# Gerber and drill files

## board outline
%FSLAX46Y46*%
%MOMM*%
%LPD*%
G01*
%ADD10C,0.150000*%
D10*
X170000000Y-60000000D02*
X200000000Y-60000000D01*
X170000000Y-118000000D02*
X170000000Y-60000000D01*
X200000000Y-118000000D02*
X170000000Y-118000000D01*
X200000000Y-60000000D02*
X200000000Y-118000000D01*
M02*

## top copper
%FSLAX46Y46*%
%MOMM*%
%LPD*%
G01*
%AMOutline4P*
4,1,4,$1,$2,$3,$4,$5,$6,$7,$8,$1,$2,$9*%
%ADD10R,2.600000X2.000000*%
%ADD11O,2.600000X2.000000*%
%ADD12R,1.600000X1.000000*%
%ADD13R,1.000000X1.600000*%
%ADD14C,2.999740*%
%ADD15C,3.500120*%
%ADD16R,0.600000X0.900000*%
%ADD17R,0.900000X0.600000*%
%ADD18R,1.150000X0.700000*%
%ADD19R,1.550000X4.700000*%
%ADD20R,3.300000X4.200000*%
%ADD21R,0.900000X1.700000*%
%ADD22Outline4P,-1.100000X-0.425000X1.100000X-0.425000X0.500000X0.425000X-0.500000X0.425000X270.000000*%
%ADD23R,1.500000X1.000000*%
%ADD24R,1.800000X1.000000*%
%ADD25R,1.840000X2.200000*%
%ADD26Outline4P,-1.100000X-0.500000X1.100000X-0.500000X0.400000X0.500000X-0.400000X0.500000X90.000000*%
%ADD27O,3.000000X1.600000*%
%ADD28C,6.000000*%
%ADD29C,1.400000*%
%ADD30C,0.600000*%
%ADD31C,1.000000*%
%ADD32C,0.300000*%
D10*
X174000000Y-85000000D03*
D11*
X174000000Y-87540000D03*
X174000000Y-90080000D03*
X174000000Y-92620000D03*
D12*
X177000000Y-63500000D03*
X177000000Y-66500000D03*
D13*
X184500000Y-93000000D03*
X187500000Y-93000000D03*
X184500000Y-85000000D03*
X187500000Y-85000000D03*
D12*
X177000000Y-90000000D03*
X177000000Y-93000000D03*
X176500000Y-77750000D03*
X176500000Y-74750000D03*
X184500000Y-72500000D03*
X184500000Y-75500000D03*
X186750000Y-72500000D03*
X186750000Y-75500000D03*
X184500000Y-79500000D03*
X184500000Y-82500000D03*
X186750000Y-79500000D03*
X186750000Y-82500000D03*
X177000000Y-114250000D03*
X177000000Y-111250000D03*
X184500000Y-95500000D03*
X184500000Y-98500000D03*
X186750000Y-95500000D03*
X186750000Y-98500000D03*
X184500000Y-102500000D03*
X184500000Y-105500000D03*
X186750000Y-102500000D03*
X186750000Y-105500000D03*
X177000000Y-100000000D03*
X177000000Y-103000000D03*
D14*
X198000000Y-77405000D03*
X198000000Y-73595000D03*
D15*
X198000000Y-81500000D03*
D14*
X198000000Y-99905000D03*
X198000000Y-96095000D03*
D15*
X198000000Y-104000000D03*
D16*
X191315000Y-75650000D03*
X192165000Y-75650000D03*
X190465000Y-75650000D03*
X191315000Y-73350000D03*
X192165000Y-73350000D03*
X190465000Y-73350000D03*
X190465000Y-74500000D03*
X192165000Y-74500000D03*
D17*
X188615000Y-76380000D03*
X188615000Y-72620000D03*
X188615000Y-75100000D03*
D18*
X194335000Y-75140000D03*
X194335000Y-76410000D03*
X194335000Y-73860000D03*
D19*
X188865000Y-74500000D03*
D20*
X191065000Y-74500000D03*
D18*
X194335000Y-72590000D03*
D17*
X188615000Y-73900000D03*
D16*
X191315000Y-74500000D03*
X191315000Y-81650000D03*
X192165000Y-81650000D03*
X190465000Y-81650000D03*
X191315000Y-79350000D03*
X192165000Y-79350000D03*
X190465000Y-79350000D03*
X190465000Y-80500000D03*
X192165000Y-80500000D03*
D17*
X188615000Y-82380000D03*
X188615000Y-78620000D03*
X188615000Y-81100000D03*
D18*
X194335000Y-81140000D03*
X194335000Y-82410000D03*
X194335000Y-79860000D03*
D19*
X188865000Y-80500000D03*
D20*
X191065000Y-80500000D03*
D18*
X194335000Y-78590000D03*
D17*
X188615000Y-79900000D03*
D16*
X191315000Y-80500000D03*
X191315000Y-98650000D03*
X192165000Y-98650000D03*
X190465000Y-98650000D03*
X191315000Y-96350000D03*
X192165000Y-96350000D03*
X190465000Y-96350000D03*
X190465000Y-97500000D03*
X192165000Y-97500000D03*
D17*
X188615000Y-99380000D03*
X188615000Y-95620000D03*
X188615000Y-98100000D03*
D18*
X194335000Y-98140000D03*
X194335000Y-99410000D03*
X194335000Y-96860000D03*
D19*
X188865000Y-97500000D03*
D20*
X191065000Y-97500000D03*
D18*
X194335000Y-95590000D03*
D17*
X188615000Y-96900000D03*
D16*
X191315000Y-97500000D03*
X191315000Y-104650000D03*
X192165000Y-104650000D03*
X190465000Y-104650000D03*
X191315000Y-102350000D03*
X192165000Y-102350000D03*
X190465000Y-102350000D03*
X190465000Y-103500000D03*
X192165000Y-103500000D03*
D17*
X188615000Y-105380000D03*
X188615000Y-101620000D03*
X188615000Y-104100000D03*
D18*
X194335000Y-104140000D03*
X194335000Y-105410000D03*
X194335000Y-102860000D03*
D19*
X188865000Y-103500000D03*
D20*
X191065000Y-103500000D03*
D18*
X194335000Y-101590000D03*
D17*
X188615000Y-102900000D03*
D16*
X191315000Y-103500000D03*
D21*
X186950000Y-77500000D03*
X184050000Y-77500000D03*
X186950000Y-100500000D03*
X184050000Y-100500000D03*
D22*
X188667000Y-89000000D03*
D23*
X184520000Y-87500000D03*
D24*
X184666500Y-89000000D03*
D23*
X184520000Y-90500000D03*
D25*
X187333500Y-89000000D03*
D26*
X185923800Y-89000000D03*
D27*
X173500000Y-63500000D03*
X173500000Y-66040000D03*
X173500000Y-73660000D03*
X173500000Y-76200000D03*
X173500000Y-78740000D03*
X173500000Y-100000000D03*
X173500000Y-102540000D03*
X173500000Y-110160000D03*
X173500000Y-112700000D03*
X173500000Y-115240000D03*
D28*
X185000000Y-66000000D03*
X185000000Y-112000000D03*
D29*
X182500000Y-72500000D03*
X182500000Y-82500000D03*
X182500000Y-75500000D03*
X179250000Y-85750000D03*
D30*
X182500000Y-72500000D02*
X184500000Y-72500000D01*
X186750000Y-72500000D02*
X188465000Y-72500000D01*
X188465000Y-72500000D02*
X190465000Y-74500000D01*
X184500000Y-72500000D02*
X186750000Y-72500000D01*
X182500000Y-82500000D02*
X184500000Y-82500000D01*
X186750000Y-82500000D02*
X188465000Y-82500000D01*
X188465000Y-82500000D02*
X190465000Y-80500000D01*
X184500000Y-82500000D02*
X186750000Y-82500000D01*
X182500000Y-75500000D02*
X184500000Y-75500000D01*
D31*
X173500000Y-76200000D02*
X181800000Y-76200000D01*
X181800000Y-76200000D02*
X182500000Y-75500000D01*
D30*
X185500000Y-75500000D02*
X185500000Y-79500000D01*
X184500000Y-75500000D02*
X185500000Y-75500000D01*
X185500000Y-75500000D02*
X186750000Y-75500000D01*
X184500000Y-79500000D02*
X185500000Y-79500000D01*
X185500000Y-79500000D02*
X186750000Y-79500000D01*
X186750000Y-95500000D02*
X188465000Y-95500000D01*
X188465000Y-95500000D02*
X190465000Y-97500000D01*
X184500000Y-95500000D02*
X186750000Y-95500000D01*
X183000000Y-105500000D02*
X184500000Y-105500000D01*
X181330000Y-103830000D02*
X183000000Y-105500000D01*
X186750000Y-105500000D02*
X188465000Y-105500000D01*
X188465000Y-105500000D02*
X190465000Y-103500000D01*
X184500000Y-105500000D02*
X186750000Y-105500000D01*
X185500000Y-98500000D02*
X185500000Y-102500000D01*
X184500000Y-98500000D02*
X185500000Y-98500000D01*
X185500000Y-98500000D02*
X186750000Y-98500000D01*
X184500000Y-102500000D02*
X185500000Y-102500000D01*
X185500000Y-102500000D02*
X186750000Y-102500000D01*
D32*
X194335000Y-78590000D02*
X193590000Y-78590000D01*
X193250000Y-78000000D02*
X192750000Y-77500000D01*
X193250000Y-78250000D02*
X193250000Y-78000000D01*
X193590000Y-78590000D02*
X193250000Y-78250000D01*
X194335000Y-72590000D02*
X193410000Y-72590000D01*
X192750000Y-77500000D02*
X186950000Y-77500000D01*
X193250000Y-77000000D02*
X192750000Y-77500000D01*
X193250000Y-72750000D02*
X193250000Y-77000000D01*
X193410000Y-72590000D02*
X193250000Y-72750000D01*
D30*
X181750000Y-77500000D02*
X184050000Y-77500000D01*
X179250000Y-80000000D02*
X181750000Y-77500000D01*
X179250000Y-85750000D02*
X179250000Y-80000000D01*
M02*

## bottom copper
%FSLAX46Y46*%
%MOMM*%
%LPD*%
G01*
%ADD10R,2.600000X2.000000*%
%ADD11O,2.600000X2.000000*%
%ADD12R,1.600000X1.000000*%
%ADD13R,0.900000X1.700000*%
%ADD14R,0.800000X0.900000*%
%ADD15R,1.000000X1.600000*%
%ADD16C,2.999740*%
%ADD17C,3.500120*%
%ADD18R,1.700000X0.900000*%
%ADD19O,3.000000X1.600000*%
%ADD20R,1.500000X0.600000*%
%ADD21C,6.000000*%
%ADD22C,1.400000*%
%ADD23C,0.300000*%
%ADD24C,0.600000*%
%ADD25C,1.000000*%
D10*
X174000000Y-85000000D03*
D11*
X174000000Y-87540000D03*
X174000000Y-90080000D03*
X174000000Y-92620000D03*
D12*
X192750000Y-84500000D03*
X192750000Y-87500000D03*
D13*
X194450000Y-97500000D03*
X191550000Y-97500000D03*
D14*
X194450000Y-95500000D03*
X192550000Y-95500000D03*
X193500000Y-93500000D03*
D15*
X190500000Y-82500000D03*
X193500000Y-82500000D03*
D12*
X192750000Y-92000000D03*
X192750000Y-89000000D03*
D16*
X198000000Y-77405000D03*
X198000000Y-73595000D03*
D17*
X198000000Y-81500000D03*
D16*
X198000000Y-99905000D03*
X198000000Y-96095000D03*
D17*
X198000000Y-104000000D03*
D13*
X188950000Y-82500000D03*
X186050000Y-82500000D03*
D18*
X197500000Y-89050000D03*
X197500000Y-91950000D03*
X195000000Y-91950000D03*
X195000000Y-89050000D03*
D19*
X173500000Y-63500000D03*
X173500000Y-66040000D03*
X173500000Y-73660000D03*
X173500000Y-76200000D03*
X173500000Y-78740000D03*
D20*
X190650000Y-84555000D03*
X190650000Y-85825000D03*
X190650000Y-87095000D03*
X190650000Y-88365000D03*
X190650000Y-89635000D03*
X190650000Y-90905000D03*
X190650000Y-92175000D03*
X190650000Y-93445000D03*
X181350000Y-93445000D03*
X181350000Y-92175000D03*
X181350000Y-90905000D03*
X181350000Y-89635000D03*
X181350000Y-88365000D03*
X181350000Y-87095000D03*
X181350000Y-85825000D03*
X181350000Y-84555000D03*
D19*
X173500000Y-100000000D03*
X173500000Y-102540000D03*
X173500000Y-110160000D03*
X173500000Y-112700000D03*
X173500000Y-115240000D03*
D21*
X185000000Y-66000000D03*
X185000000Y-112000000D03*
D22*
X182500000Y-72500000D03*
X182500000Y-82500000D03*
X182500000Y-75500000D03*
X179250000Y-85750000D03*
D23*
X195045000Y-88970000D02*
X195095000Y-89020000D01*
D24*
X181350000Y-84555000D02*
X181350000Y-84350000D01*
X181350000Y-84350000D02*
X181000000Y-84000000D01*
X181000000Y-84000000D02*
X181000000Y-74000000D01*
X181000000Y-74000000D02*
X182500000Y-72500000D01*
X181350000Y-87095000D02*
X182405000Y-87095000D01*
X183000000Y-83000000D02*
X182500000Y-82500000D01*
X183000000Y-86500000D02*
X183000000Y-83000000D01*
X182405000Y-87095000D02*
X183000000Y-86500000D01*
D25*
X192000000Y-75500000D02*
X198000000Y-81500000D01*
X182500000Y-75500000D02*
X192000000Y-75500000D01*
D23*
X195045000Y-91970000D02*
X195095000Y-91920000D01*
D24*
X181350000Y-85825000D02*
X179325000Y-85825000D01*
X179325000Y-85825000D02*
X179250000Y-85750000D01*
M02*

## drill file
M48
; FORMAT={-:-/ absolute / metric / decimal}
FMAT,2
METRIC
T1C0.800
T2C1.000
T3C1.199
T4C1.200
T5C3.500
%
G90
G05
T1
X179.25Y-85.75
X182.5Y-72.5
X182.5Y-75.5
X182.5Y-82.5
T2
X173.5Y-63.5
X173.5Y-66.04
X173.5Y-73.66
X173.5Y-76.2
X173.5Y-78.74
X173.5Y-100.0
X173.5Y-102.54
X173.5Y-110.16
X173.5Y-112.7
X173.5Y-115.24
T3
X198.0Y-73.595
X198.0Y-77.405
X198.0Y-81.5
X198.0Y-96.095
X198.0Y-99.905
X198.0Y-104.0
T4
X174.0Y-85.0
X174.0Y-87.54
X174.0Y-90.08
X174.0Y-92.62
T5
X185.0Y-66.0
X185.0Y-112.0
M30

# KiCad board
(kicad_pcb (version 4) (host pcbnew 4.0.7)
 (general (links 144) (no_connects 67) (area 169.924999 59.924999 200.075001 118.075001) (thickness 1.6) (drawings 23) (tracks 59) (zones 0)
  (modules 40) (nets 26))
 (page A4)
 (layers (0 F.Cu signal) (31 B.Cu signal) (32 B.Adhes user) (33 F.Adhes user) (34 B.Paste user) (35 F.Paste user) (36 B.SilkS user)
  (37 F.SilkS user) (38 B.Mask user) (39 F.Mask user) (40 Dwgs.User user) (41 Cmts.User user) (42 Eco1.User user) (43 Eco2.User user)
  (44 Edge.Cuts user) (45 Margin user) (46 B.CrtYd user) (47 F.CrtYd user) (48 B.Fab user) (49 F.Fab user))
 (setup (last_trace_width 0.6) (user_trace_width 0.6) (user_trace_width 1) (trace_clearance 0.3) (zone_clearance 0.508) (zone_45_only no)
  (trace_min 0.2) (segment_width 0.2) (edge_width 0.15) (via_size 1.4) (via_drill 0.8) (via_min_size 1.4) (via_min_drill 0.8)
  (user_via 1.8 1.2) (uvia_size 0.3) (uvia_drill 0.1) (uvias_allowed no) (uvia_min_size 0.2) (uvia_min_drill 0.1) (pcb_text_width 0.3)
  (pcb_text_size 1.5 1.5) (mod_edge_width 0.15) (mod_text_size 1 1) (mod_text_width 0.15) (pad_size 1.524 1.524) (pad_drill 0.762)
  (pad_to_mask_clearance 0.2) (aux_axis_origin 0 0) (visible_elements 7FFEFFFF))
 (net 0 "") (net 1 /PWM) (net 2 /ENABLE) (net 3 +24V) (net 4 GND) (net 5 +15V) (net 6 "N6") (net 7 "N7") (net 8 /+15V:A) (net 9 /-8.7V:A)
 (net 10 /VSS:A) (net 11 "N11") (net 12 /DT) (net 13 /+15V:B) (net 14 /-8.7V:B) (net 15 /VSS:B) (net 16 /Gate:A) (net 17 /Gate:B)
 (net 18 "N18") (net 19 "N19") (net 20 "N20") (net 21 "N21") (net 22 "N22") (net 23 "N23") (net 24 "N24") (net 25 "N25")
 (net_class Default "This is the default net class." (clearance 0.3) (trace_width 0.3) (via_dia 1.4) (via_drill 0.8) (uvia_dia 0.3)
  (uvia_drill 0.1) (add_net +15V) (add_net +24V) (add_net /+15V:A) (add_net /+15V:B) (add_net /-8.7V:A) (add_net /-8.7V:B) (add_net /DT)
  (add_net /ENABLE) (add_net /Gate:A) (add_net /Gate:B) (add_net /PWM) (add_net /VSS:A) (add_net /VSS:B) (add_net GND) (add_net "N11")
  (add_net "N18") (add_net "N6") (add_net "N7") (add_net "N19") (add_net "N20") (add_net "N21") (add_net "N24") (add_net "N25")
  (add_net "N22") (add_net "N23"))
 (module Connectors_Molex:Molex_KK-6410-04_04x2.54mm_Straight (layer B.Cu) (at 174 85 270)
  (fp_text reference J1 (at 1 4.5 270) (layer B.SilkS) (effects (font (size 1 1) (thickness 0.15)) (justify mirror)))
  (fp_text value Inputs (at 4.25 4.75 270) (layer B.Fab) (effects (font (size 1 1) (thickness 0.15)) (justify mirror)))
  (pad 1 thru_hole rect (at 0 0 270) (size 2 2.6) (drill 1.2) (layers *.Cu *.Mask) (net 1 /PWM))
  (pad 2 thru_hole oval (at 2.54 0 270) (size 2 2.6) (drill 1.2) (layers *.Cu *.Mask) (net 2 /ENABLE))
  (pad 3 thru_hole oval (at 5.08 0 270) (size 2 2.6) (drill 1.2) (layers *.Cu *.Mask) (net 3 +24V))
  (pad 4 thru_hole oval (at 7.62 0 270) (size 2 2.6) (drill 1.2) (layers *.Cu *.Mask) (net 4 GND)))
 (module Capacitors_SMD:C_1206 (layer B.Cu) (at 192.75 86 270)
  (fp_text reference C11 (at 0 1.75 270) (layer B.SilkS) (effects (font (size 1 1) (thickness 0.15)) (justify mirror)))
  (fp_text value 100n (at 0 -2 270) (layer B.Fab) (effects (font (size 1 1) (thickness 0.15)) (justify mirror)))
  (pad 1 smd rect (at -1.5 0 270) (size 1 1.6) (layers B.Cu B.Paste B.Mask) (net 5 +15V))
  (pad 2 smd rect (at 1.5 0 270) (size 1 1.6) (layers B.Cu B.Paste B.Mask) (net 4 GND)))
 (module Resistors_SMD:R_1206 (layer B.Cu) (at 193 97.5 180)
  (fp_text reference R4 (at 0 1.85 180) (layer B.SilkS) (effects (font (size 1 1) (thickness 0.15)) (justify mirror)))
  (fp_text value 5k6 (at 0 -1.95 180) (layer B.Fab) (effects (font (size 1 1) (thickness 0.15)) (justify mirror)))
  (pad 1 smd rect (at -1.45 0 180) (size 0.9 1.7) (layers B.Cu B.Paste B.Mask) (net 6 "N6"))
  (pad 2 smd rect (at 1.45 0 180) (size 0.9 1.7) (layers B.Cu B.Paste B.Mask) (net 2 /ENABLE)))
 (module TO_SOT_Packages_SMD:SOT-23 (layer B.Cu) (at 193.5 94.5 90)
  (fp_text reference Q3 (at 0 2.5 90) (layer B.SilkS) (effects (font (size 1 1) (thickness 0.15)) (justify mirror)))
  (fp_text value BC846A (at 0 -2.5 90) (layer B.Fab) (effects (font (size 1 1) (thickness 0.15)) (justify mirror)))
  (pad 1 smd rect (at -1 0.95 90) (size 0.9 0.8) (layers B.Cu B.Paste B.Mask) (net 6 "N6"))
  (pad 2 smd rect (at -1 -0.95 90) (size 0.9 0.8) (layers B.Cu B.Paste B.Mask) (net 4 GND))
  (pad 3 smd rect (at 1 0 90) (size 0.9 0.8) (layers B.Cu B.Paste B.Mask) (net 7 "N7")))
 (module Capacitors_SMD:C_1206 (layer F.Cu) (at 177 65 270)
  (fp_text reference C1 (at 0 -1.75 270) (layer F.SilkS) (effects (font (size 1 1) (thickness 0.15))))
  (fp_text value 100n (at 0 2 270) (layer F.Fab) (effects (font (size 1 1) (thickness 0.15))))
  (pad 1 smd rect (at -1.5 0 270) (size 1 1.6) (layers F.Cu F.Paste F.Mask) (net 3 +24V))
  (pad 2 smd rect (at 1.5 0 270) (size 1 1.6) (layers F.Cu F.Paste F.Mask) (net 4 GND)))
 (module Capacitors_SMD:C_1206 (layer F.Cu) (at 186 93)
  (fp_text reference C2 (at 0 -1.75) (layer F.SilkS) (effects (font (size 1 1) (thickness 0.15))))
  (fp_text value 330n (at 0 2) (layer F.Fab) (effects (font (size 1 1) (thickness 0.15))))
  (pad 1 smd rect (at -1.5 0) (size 1 1.6) (layers F.Cu F.Paste F.Mask) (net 3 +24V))
  (pad 2 smd rect (at 1.5 0) (size 1 1.6) (layers F.Cu F.Paste F.Mask) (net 4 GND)))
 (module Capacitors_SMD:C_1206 (layer F.Cu) (at 186 85)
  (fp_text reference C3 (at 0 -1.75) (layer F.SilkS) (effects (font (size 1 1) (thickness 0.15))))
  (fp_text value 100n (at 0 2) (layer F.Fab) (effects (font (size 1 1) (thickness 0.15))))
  (pad 1 smd rect (at -1.5 0) (size 1 1.6) (layers F.Cu F.Paste F.Mask) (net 5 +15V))
  (pad 2 smd rect (at 1.5 0) (size 1 1.6) (layers F.Cu F.Paste F.Mask) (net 4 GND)))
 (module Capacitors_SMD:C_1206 (layer F.Cu) (at 177 91.5 270)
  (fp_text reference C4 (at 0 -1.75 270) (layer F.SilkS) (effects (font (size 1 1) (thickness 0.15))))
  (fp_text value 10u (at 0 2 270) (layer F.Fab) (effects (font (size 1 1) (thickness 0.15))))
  (pad 1 smd rect (at -1.5 0 270) (size 1 1.6) (layers F.Cu F.Paste F.Mask) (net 3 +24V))
  (pad 2 smd rect (at 1.5 0 270) (size 1 1.6) (layers F.Cu F.Paste F.Mask) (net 4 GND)))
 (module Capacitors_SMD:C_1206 (layer F.Cu) (at 176.5 76.25 90)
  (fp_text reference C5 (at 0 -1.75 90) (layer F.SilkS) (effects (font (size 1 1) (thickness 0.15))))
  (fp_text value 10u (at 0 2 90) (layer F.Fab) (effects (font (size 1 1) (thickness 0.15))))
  (pad 1 smd rect (at -1.5 0 90) (size 1 1.6) (layers F.Cu F.Paste F.Mask) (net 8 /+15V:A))
  (pad 2 smd rect (at 1.5 0 90) (size 1 1.6) (layers F.Cu F.Paste F.Mask) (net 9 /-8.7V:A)))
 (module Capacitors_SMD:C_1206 (layer F.Cu) (at 184.5 74 270)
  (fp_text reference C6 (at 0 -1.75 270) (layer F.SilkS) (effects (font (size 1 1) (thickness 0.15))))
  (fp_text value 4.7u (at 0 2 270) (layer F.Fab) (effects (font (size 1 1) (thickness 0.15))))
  (pad 1 smd rect (at -1.5 0 270) (size 1 1.6) (layers F.Cu F.Paste F.Mask) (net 8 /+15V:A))
  (pad 2 smd rect (at 1.5 0 270) (size 1 1.6) (layers F.Cu F.Paste F.Mask) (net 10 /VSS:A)))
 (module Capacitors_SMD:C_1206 (layer F.Cu) (at 186.75 74 270)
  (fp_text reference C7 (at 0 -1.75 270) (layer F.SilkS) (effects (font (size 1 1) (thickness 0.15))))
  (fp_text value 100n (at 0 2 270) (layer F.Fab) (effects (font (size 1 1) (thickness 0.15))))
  (pad 1 smd rect (at -1.5 0 270) (size 1 1.6) (layers F.Cu F.Paste F.Mask) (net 8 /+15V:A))
  (pad 2 smd rect (at 1.5 0 270) (size 1 1.6) (layers F.Cu F.Paste F.Mask) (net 10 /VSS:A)))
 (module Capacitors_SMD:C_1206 (layer B.Cu) (at 192 82.5)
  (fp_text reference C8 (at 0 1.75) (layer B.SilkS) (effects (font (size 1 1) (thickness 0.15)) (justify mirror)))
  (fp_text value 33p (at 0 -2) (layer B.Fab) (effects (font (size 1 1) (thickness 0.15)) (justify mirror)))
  (pad 1 smd rect (at -1.5 0) (size 1 1.6) (layers B.Cu B.Paste B.Mask) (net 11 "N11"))
  (pad 2 smd rect (at 1.5 0) (size 1 1.6) (layers B.Cu B.Paste B.Mask) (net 4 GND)))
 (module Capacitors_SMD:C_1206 (layer F.Cu) (at 184.5 81 270)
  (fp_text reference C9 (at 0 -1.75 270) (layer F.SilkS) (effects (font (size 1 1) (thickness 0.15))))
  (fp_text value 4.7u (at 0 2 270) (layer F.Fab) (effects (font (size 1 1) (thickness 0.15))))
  (pad 1 smd rect (at -1.5 0 270) (size 1 1.6) (layers F.Cu F.Paste F.Mask) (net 10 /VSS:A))
  (pad 2 smd rect (at 1.5 0 270) (size 1 1.6) (layers F.Cu F.Paste F.Mask) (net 9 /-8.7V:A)))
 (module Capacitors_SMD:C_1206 (layer F.Cu) (at 186.75 81 270)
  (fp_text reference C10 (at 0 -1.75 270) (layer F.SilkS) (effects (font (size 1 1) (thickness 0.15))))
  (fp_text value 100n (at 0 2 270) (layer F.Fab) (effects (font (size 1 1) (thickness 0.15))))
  (pad 1 smd rect (at -1.5 0 270) (size 1 1.6) (layers F.Cu F.Paste F.Mask) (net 10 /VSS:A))
  (pad 2 smd rect (at 1.5 0 270) (size 1 1.6) (layers F.Cu F.Paste F.Mask) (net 9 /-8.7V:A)))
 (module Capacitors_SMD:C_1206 (layer B.Cu) (at 192.75 90.5 90)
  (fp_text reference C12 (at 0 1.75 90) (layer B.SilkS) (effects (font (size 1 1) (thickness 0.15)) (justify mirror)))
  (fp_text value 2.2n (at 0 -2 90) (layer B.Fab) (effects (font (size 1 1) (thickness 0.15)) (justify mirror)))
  (pad 1 smd rect (at -1.5 0 90) (size 1 1.6) (layers B.Cu B.Paste B.Mask) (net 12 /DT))
  (pad 2 smd rect (at 1.5 0 90) (size 1 1.6) (layers B.Cu B.Paste B.Mask) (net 4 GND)))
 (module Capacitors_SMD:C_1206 (layer F.Cu) (at 177 112.75 90)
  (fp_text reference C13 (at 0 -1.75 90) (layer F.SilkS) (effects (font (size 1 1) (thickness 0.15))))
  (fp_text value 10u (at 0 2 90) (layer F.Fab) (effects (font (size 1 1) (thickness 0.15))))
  (pad 1 smd rect (at -1.5 0 90) (size 1 1.6) (layers F.Cu F.Paste F.Mask) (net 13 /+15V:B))
  (pad 2 smd rect (at 1.5 0 90) (size 1 1.6) (layers F.Cu F.Paste F.Mask) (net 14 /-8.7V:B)))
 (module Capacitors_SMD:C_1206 (layer F.Cu) (at 184.5 97 270)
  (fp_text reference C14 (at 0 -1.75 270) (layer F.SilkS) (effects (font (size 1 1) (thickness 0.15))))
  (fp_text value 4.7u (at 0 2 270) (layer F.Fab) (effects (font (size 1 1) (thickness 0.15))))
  (pad 1 smd rect (at -1.5 0 270) (size 1 1.6) (layers F.Cu F.Paste F.Mask) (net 13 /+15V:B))
  (pad 2 smd rect (at 1.5 0 270) (size 1 1.6) (layers F.Cu F.Paste F.Mask) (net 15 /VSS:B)))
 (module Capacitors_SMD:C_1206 (layer F.Cu) (at 186.75 97 270)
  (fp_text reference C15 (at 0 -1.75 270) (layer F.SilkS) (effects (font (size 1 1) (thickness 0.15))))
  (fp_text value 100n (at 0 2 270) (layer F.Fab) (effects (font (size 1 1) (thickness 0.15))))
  (pad 1 smd rect (at -1.5 0 270) (size 1 1.6) (layers F.Cu F.Paste F.Mask) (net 13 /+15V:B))
  (pad 2 smd rect (at 1.5 0 270) (size 1 1.6) (layers F.Cu F.Paste F.Mask) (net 15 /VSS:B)))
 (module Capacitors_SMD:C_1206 (layer F.Cu) (at 184.5 104 270)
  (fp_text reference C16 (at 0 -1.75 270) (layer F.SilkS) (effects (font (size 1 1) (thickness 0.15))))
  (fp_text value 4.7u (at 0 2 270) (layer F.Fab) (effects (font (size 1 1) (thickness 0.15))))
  (pad 1 smd rect (at -1.5 0 270) (size 1 1.6) (layers F.Cu F.Paste F.Mask) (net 15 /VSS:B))
  (pad 2 smd rect (at 1.5 0 270) (size 1 1.6) (layers F.Cu F.Paste F.Mask) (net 14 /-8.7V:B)))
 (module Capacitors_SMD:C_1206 (layer F.Cu) (at 186.75 104 270)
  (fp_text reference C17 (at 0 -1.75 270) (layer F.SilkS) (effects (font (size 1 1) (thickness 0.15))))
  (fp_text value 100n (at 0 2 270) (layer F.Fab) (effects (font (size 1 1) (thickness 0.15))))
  (pad 1 smd rect (at -1.5 0 270) (size 1 1.6) (layers F.Cu F.Paste F.Mask) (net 15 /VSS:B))
  (pad 2 smd rect (at 1.5 0 270) (size 1 1.6) (layers F.Cu F.Paste F.Mask) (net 14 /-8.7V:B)))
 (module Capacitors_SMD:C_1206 (layer F.Cu) (at 177 101.5 270)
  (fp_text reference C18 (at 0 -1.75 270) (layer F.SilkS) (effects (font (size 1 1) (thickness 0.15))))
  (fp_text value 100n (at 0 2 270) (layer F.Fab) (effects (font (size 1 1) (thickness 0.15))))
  (pad 1 smd rect (at -1.5 0 270) (size 1 1.6) (layers F.Cu F.Paste F.Mask) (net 3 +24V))
  (pad 2 smd rect (at 1.5 0 270) (size 1 1.6) (layers F.Cu F.Paste F.Mask) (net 4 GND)))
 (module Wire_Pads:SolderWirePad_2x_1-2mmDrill (layer F.Cu) (at 198 75.5 90)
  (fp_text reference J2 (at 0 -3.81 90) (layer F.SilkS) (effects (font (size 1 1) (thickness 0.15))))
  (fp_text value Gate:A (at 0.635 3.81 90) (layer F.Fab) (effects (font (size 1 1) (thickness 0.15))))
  (pad 1 thru_hole circle (at -1.905 0 90) (size 2.99974 2.99974) (drill 1.19888) (layers *.Cu *.Mask) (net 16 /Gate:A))
  (pad 1 thru_hole circle (at 1.905 0 90) (size 2.99974 2.99974) (drill 1.19888) (layers *.Cu *.Mask) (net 16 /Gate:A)))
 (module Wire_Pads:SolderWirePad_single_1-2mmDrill (layer F.Cu) (at 198 81.5)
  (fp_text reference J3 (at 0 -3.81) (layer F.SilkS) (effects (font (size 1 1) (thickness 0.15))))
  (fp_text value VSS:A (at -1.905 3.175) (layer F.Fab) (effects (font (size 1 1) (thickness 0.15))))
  (pad 1 thru_hole circle (at 0 0) (size 3.50012 3.50012) (drill 1.19888) (layers *.Cu *.Mask) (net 10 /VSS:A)))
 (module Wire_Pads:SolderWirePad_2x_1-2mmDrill (layer F.Cu) (at 198 98 90)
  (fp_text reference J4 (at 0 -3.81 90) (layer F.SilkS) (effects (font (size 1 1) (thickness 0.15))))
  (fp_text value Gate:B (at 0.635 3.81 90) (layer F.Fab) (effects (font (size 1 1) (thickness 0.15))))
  (pad 1 thru_hole circle (at -1.905 0 90) (size 2.99974 2.99974) (drill 1.19888) (layers *.Cu *.Mask) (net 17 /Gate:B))
  (pad 1 thru_hole circle (at 1.905 0 90) (size 2.99974 2.99974) (drill 1.19888) (layers *.Cu *.Mask) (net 17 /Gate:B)))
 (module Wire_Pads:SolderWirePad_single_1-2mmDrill (layer F.Cu) (at 198 104)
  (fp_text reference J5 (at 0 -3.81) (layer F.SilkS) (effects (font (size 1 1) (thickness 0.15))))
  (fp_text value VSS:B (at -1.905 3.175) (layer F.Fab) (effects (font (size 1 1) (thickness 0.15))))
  (pad 1 thru_hole circle (at 0 0) (size 3.50012 3.50012) (drill 1.19888) (layers *.Cu *.Mask) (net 15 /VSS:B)))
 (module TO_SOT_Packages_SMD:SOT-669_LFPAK (layer F.Cu) (at 191.5 74.5 180) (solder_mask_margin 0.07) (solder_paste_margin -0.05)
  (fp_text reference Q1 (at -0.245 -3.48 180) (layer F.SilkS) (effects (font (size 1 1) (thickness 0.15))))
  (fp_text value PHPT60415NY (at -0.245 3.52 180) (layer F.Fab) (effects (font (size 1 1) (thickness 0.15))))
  (pad 5 smd rect (at 0.185 -1.15 180) (size 0.6 0.9) (layers F.Cu F.Paste F.Mask) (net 8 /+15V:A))
  (pad 5 smd rect (at -0.665 -1.15 180) (size 0.6 0.9) (layers F.Cu F.Paste F.Mask) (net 8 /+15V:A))
  (pad 5 smd rect (at 1.035 -1.15 180) (size 0.6 0.9) (layers F.Cu F.Paste F.Mask) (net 8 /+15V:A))
  (pad 5 smd rect (at 0.185 1.15 180) (size 0.6 0.9) (layers F.Cu F.Paste F.Mask) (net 8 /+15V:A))
  (pad 5 smd rect (at -0.665 1.15 180) (size 0.6 0.9) (layers F.Cu F.Paste F.Mask) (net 8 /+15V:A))
  (pad 5 smd rect (at 1.035 1.15 180) (size 0.6 0.9) (layers F.Cu F.Paste F.Mask) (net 8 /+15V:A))
  (pad 5 smd rect (at 1.035 0 180) (size 0.6 0.9) (layers F.Cu F.Paste F.Mask) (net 8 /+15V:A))
  (pad 5 smd rect (at -0.665 0 180) (size 0.6 0.9) (layers F.Cu F.Paste F.Mask) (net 8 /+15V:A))
  (pad 5 smd rect (at 2.885 -1.88 90) (size 0.6 0.9) (layers F.Cu F.Paste F.Mask) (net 8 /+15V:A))
  (pad 5 smd rect (at 2.885 1.88 90) (size 0.6 0.9) (layers F.Cu F.Paste F.Mask) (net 8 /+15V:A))
  (pad 5 smd rect (at 2.885 -0.6 90) (size 0.6 0.9) (layers F.Cu F.Paste F.Mask) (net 8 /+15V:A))
  (pad 2 smd rect (at -2.835 -0.64 90) (size 0.7 1.15) (layers F.Cu F.Paste F.Mask) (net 16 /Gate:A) (solder_mask_margin 0.07)
   (solder_paste_margin -0.05))
  (pad 1 smd rect (at -2.835 -1.91 90) (size 0.7 1.15) (layers F.Cu F.Paste F.Mask) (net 16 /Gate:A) (solder_mask_margin 0.07)
   (solder_paste_margin -0.05))
  (pad 3 smd rect (at -2.835 0.64 90) (size 0.7 1.15) (layers F.Cu F.Paste F.Mask) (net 16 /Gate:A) (solder_mask_margin 0.07)
   (solder_paste_margin -0.05))
  (pad 5 smd rect (at 2.635 0 90) (size 4.7 1.55) (layers F.Cu F.Paste F.Mask) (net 8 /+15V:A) (solder_mask_margin 0.07))
  (pad 5 smd rect (at 0.435 0 90) (size 4.2 3.3) (layers F.Cu F.Paste F.Mask) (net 8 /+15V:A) (solder_mask_margin 0.07))
  (pad 4 smd rect (at -2.835 1.91 90) (size 0.7 1.15) (layers F.Cu F.Paste F.Mask) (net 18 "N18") (solder_mask_margin 0.07)
   (solder_paste_margin -0.05))
  (pad 5 smd rect (at 2.885 0.6 90) (size 0.6 0.9) (layers F.Cu F.Paste F.Mask) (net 8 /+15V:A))
  (pad 5 smd rect (at 0.185 0 180) (size 0.6 0.9) (layers F.Cu F.Paste F.Mask) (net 8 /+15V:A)))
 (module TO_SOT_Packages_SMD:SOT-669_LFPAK (layer F.Cu) (at 191.5 80.5 180) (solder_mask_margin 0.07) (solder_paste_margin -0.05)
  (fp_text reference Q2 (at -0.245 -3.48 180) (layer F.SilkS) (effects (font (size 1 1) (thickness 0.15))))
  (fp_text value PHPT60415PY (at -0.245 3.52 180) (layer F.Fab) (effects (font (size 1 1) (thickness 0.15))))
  (pad 5 smd rect (at 0.185 -1.15 180) (size 0.6 0.9) (layers F.Cu F.Paste F.Mask) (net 9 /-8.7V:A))
  (pad 5 smd rect (at -0.665 -1.15 180) (size 0.6 0.9) (layers F.Cu F.Paste F.Mask) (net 9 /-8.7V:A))
  (pad 5 smd rect (at 1.035 -1.15 180) (size 0.6 0.9) (layers F.Cu F.Paste F.Mask) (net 9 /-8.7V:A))
  (pad 5 smd rect (at 0.185 1.15 180) (size 0.6 0.9) (layers F.Cu F.Paste F.Mask) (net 9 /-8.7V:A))
  (pad 5 smd rect (at -0.665 1.15 180) (size 0.6 0.9) (layers F.Cu F.Paste F.Mask) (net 9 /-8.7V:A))
  (pad 5 smd rect (at 1.035 1.15 180) (size 0.6 0.9) (layers F.Cu F.Paste F.Mask) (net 9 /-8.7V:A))
  (pad 5 smd rect (at 1.035 0 180) (size 0.6 0.9) (layers F.Cu F.Paste F.Mask) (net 9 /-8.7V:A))
  (pad 5 smd rect (at -0.665 0 180) (size 0.6 0.9) (layers F.Cu F.Paste F.Mask) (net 9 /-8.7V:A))
  (pad 5 smd rect (at 2.885 -1.88 90) (size 0.6 0.9) (layers F.Cu F.Paste F.Mask) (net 9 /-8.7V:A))
  (pad 5 smd rect (at 2.885 1.88 90) (size 0.6 0.9) (layers F.Cu F.Paste F.Mask) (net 9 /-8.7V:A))
  (pad 5 smd rect (at 2.885 -0.6 90) (size 0.6 0.9) (layers F.Cu F.Paste F.Mask) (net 9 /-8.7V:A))
  (pad 2 smd rect (at -2.835 -0.64 90) (size 0.7 1.15) (layers F.Cu F.Paste F.Mask) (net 16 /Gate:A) (solder_mask_margin 0.07)
   (solder_paste_margin -0.05))
  (pad 1 smd rect (at -2.835 -1.91 90) (size 0.7 1.15) (layers F.Cu F.Paste F.Mask) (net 16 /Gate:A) (solder_mask_margin 0.07)
   (solder_paste_margin -0.05))
  (pad 3 smd rect (at -2.835 0.64 90) (size 0.7 1.15) (layers F.Cu F.Paste F.Mask) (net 16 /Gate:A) (solder_mask_margin 0.07)
   (solder_paste_margin -0.05))
  (pad 5 smd rect (at 2.635 0 90) (size 4.7 1.55) (layers F.Cu F.Paste F.Mask) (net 9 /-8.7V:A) (solder_mask_margin 0.07))
  (pad 5 smd rect (at 0.435 0 90) (size 4.2 3.3) (layers F.Cu F.Paste F.Mask) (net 9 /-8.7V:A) (solder_mask_margin 0.07))
  (pad 4 smd rect (at -2.835 1.91 90) (size 0.7 1.15) (layers F.Cu F.Paste F.Mask) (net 18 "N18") (solder_mask_margin 0.07)
   (solder_paste_margin -0.05))
  (pad 5 smd rect (at 2.885 0.6 90) (size 0.6 0.9) (layers F.Cu F.Paste F.Mask) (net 9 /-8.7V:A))
  (pad 5 smd rect (at 0.185 0 180) (size 0.6 0.9) (layers F.Cu F.Paste F.Mask) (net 9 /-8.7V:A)))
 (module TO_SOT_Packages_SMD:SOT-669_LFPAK (layer F.Cu) (at 191.5 97.5 180) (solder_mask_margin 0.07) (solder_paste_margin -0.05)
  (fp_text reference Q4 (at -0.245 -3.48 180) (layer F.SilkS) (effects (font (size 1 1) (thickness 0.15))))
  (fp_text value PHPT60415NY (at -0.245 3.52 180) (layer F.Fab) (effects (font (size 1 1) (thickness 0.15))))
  (pad 5 smd rect (at 0.185 -1.15 180) (size 0.6 0.9) (layers F.Cu F.Paste F.Mask) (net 13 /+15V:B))
  (pad 5 smd rect (at -0.665 -1.15 180) (size 0.6 0.9) (layers F.Cu F.Paste F.Mask) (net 13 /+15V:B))
  (pad 5 smd rect (at 1.035 -1.15 180) (size 0.6 0.9) (layers F.Cu F.Paste F.Mask) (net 13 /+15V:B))
  (pad 5 smd rect (at 0.185 1.15 180) (size 0.6 0.9) (layers F.Cu F.Paste F.Mask) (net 13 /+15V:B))
  (pad 5 smd rect (at -0.665 1.15 180) (size 0.6 0.9) (layers F.Cu F.Paste F.Mask) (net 13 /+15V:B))
  (pad 5 smd rect (at 1.035 1.15 180) (size 0.6 0.9) (layers F.Cu F.Paste F.Mask) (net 13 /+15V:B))
  (pad 5 smd rect (at 1.035 0 180) (size 0.6 0.9) (layers F.Cu F.Paste F.Mask) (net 13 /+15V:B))
  (pad 5 smd rect (at -0.665 0 180) (size 0.6 0.9) (layers F.Cu F.Paste F.Mask) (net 13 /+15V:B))
  (pad 5 smd rect (at 2.885 -1.88 90) (size 0.6 0.9) (layers F.Cu F.Paste F.Mask) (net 13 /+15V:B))
  (pad 5 smd rect (at 2.885 1.88 90) (size 0.6 0.9) (layers F.Cu F.Paste F.Mask) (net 13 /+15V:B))
  (pad 5 smd rect (at 2.885 -0.6 90) (size 0.6 0.9) (layers F.Cu F.Paste F.Mask) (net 13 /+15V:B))
  (pad 2 smd rect (at -2.835 -0.64 90) (size 0.7 1.15) (layers F.Cu F.Paste F.Mask) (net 17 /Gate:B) (solder_mask_margin 0.07)
   (solder_paste_margin -0.05))
  (pad 1 smd rect (at -2.835 -1.91 90) (size 0.7 1.15) (layers F.Cu F.Paste F.Mask) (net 17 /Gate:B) (solder_mask_margin 0.07)
   (solder_paste_margin -0.05))
  (pad 3 smd rect (at -2.835 0.64 90) (size 0.7 1.15) (layers F.Cu F.Paste F.Mask) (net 17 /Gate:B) (solder_mask_margin 0.07)
   (solder_paste_margin -0.05))
  (pad 5 smd rect (at 2.635 0 90) (size 4.7 1.55) (layers F.Cu F.Paste F.Mask) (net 13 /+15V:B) (solder_mask_margin 0.07))
  (pad 5 smd rect (at 0.435 0 90) (size 4.2 3.3) (layers F.Cu F.Paste F.Mask) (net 13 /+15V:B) (solder_mask_margin 0.07))
  (pad 4 smd rect (at -2.835 1.91 90) (size 0.7 1.15) (layers F.Cu F.Paste F.Mask) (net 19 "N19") (solder_mask_margin 0.07)
   (solder_paste_margin -0.05))
  (pad 5 smd rect (at 2.885 0.6 90) (size 0.6 0.9) (layers F.Cu F.Paste F.Mask) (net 13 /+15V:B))
  (pad 5 smd rect (at 0.185 0 180) (size 0.6 0.9) (layers F.Cu F.Paste F.Mask) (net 13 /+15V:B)))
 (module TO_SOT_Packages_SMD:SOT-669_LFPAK (layer F.Cu) (at 191.5 103.5 180) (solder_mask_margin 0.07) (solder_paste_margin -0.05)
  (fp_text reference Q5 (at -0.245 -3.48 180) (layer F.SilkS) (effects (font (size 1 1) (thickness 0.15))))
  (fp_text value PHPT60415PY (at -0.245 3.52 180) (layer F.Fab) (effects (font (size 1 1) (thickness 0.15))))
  (pad 5 smd rect (at 0.185 -1.15 180) (size 0.6 0.9) (layers F.Cu F.Paste F.Mask) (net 14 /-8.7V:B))
  (pad 5 smd rect (at -0.665 -1.15 180) (size 0.6 0.9) (layers F.Cu F.Paste F.Mask) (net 14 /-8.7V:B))
  (pad 5 smd rect (at 1.035 -1.15 180) (size 0.6 0.9) (layers F.Cu F.Paste F.Mask) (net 14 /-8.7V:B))
  (pad 5 smd rect (at 0.185 1.15 180) (size 0.6 0.9) (layers F.Cu F.Paste F.Mask) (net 14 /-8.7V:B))
  (pad 5 smd rect (at -0.665 1.15 180) (size 0.6 0.9) (layers F.Cu F.Paste F.Mask) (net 14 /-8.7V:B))
  (pad 5 smd rect (at 1.035 1.15 180) (size 0.6 0.9) (layers F.Cu F.Paste F.Mask) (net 14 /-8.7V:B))
  (pad 5 smd rect (at 1.035 0 180) (size 0.6 0.9) (layers F.Cu F.Paste F.Mask) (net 14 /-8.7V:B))
  (pad 5 smd rect (at -0.665 0 180) (size 0.6 0.9) (layers F.Cu F.Paste F.Mask) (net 14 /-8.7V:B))
  (pad 5 smd rect (at 2.885 -1.88 90) (size 0.6 0.9) (layers F.Cu F.Paste F.Mask) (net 14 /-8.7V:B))
  (pad 5 smd rect (at 2.885 1.88 90) (size 0.6 0.9) (layers F.Cu F.Paste F.Mask) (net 14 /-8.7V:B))
  (pad 5 smd rect (at 2.885 -0.6 90) (size 0.6 0.9) (layers F.Cu F.Paste F.Mask) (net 14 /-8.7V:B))
  (pad 2 smd rect (at -2.835 -0.64 90) (size 0.7 1.15) (layers F.Cu F.Paste F.Mask) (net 17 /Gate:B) (solder_mask_margin 0.07)
   (solder_paste_margin -0.05))
  (pad 1 smd rect (at -2.835 -1.91 90) (size 0.7 1.15) (layers F.Cu F.Paste F.Mask) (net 17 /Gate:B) (solder_mask_margin 0.07)
   (solder_paste_margin -0.05))
  (pad 3 smd rect (at -2.835 0.64 90) (size 0.7 1.15) (layers F.Cu F.Paste F.Mask) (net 17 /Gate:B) (solder_mask_margin 0.07)
   (solder_paste_margin -0.05))
  (pad 5 smd rect (at 2.635 0 90) (size 4.7 1.55) (layers F.Cu F.Paste F.Mask) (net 14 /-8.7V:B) (solder_mask_margin 0.07))
  (pad 5 smd rect (at 0.435 0 90) (size 4.2 3.3) (layers F.Cu F.Paste F.Mask) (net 14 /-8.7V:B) (solder_mask_margin 0.07))
  (pad 4 smd rect (at -2.835 1.91 90) (size 0.7 1.15) (layers F.Cu F.Paste F.Mask) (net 19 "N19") (solder_mask_margin 0.07)
   (solder_paste_margin -0.05))
  (pad 5 smd rect (at 2.885 0.6 90) (size 0.6 0.9) (layers F.Cu F.Paste F.Mask) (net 14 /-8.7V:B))
  (pad 5 smd rect (at 0.185 0 180) (size 0.6 0.9) (layers F.Cu F.Paste F.Mask) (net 14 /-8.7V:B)))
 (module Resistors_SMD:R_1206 (layer B.Cu) (at 187.5 82.5 180)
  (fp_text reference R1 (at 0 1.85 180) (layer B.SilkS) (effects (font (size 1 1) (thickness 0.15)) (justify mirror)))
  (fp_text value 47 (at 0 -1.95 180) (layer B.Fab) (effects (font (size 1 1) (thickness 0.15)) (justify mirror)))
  (pad 1 smd rect (at -1.45 0 180) (size 0.9 1.7) (layers B.Cu B.Paste B.Mask) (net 11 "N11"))
  (pad 2 smd rect (at 1.45 0 180) (size 0.9 1.7) (layers B.Cu B.Paste B.Mask) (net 1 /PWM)))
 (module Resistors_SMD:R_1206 (layer F.Cu) (at 185.5 77.5 180)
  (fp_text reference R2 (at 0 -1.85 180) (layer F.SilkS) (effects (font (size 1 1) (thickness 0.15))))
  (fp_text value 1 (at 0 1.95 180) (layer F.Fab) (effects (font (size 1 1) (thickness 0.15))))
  (pad 1 smd rect (at -1.45 0 180) (size 0.9 1.7) (layers F.Cu F.Paste F.Mask) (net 18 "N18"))
  (pad 2 smd rect (at 1.45 0 180) (size 0.9 1.7) (layers F.Cu F.Paste F.Mask) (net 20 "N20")))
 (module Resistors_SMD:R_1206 (layer B.Cu) (at 197.5 90.5 270)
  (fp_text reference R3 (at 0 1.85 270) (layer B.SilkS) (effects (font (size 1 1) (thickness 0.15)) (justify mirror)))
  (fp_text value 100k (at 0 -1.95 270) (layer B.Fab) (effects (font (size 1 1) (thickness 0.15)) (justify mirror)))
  (pad 1 smd rect (at -1.45 0 270) (size 0.9 1.7) (layers B.Cu B.Paste B.Mask) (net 5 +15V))
  (pad 2 smd rect (at 1.45 0 270) (size 0.9 1.7) (layers B.Cu B.Paste B.Mask) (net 7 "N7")))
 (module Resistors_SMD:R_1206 (layer B.Cu) (at 195 90.5 90)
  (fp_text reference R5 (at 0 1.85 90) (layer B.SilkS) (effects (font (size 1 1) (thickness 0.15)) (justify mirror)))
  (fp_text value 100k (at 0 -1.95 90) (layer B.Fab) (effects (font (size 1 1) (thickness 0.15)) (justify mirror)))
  (pad 1 smd rect (at -1.45 0 90) (size 0.9 1.7) (layers B.Cu B.Paste B.Mask) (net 12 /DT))
  (pad 2 smd rect (at 1.45 0 90) (size 0.9 1.7) (layers B.Cu B.Paste B.Mask) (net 4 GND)))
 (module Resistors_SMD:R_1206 (layer F.Cu) (at 185.5 100.5 180)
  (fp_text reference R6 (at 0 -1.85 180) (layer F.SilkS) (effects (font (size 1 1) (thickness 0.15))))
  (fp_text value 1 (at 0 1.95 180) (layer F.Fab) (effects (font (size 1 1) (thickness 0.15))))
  (pad 1 smd rect (at -1.45 0 180) (size 0.9 1.7) (layers F.Cu F.Paste F.Mask) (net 19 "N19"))
  (pad 2 smd rect (at 1.45 0 180) (size 0.9 1.7) (layers F.Cu F.Paste F.Mask) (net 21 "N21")))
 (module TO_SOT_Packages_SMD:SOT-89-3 (layer F.Cu) (at 186 89)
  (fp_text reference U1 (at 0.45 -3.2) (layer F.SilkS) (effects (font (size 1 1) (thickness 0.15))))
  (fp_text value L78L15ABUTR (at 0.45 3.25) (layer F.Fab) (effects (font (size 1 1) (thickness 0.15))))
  (pad 2 smd trapezoid (at 2.667 0 270) (size 1.6 0.85) (rect_delta 0 0.6) (layers F.Cu F.Paste F.Mask) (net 4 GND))
  (pad 1 smd rect (at -1.48 -1.5 270) (size 1 1.5) (layers F.Cu F.Paste F.Mask) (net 5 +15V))
  (pad 2 smd rect (at -1.3335 0 270) (size 1 1.8) (layers F.Cu F.Paste F.Mask) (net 4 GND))
  (pad 3 smd rect (at -1.48 1.5 270) (size 1 1.5) (layers F.Cu F.Paste F.Mask) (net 3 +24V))
  (pad 2 smd rect (at 1.3335 0 270) (size 2.2 1.84) (layers F.Cu F.Paste F.Mask) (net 4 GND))
  (pad 2 smd trapezoid (at -0.0762 0 90) (size 1.5 1) (rect_delta 0 0.7) (layers F.Cu F.Paste F.Mask) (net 4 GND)))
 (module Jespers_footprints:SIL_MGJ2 (layer B.Cu) (at 173.5 63.5 270)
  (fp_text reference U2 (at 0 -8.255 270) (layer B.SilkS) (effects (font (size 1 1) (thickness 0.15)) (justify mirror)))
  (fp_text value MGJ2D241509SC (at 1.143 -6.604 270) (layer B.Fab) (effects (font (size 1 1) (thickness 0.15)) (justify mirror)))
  (pad 1 thru_hole oval (at 0 0 270) (size 1.6 3) (drill 1) (layers *.Cu *.Mask) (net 3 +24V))
  (pad 2 thru_hole oval (at 2.54 0 270) (size 1.6 3) (drill 1) (layers *.Cu *.Mask) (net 4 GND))
  (pad 5 thru_hole oval (at 10.16 0 270) (size 1.6 3) (drill 1) (layers *.Cu *.Mask) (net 9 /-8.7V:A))
  (pad 6 thru_hole oval (at 12.7 0 270) (size 1.6 3) (drill 1) (layers *.Cu *.Mask) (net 10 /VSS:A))
  (pad 7 thru_hole oval (at 15.24 0 270) (size 1.6 3) (drill 1) (layers *.Cu *.Mask) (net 8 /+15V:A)))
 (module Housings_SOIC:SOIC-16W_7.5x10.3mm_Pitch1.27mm (layer B.Cu) (at 186 89 180)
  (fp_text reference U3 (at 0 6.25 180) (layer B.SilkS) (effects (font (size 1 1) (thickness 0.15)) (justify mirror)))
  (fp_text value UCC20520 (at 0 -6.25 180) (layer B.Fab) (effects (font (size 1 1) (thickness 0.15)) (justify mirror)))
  (pad 1 smd rect (at -4.65 4.445 180) (size 1.5 0.6) (layers B.Cu B.Paste B.Mask) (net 11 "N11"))
  (pad 2 smd rect (at -4.65 3.175 180) (size 1.5 0.6) (layers B.Cu B.Paste B.Mask) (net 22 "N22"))
  (pad 3 smd rect (at -4.65 1.905 180) (size 1.5 0.6) (layers B.Cu B.Paste B.Mask) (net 5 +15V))
  (pad 4 smd rect (at -4.65 0.635 180) (size 1.5 0.6) (layers B.Cu B.Paste B.Mask) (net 4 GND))
  (pad 5 smd rect (at -4.65 -0.635 180) (size 1.5 0.6) (layers B.Cu B.Paste B.Mask) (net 7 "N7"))
  (pad 6 smd rect (at -4.65 -1.905 180) (size 1.5 0.6) (layers B.Cu B.Paste B.Mask) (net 12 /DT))
  (pad 7 smd rect (at -4.65 -3.175 180) (size 1.5 0.6) (layers B.Cu B.Paste B.Mask) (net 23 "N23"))
  (pad 8 smd rect (at -4.65 -4.445 180) (size 1.5 0.6) (layers B.Cu B.Paste B.Mask) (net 5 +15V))
  (pad 9 smd rect (at 4.65 -4.445 180) (size 1.5 0.6) (layers B.Cu B.Paste B.Mask) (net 14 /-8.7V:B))
  (pad 10 smd rect (at 4.65 -3.175 180) (size 1.5 0.6) (layers B.Cu B.Paste B.Mask) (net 21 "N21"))
  (pad 11 smd rect (at 4.65 -1.905 180) (size 1.5 0.6) (layers B.Cu B.Paste B.Mask) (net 13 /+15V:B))
  (pad 12 smd rect (at 4.65 -0.635 180) (size 1.5 0.6) (layers B.Cu B.Paste B.Mask) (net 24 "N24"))
  (pad 13 smd rect (at 4.65 0.635 180) (size 1.5 0.6) (layers B.Cu B.Paste B.Mask) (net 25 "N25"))
  (pad 14 smd rect (at 4.65 1.905 180) (size 1.5 0.6) (layers B.Cu B.Paste B.Mask) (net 9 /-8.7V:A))
  (pad 15 smd rect (at 4.65 3.175 180) (size 1.5 0.6) (layers B.Cu B.Paste B.Mask) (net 20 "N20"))
  (pad 16 smd rect (at 4.65 4.445 180) (size 1.5 0.6) (layers B.Cu B.Paste B.Mask) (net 8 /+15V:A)))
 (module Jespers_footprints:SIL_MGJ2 (layer B.Cu) (at 173.5 100 270)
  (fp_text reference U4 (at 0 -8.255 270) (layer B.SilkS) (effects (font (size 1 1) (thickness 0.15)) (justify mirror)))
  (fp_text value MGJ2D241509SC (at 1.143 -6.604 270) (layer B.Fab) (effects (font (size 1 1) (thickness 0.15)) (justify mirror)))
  (pad 1 thru_hole oval (at 0 0 270) (size 1.6 3) (drill 1) (layers *.Cu *.Mask) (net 3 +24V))
  (pad 2 thru_hole oval (at 2.54 0 270) (size 1.6 3) (drill 1) (layers *.Cu *.Mask) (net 4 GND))
  (pad 5 thru_hole oval (at 10.16 0 270) (size 1.6 3) (drill 1) (layers *.Cu *.Mask) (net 14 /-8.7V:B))
  (pad 6 thru_hole oval (at 12.7 0 270) (size 1.6 3) (drill 1) (layers *.Cu *.Mask) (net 15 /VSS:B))
  (pad 7 thru_hole oval (at 15.24 0 270) (size 1.6 3) (drill 1) (layers *.Cu *.Mask) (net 13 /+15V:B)))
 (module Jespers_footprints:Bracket (layer F.Cu) (at 200 66)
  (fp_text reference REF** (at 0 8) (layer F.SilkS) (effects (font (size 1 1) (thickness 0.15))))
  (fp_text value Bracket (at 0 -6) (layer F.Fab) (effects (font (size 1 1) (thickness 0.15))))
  (pad 1 thru_hole circle (at -15 0) (size 6 6) (drill 3.5) (layers *.Cu *.Mask)))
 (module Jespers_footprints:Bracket (layer F.Cu) (at 200 112)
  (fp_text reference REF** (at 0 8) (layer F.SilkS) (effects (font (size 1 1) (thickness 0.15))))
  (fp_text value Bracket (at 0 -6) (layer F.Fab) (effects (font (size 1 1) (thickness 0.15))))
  (pad 1 thru_hole circle (at -15 0) (size 6 6) (drill 3.5) (layers *.Cu *.Mask)))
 (gr_line (start 170 60) (end 200 60) (angle 90) (layer Edge.Cuts) (width 0.15))
 (gr_line (start 170 118) (end 170 60) (angle 90) (layer Edge.Cuts) (width 0.15))
 (gr_line (start 200 118) (end 170 118) (angle 90) (layer Edge.Cuts) (width 0.15))
 (gr_line (start 200 60) (end 200 118) (angle 90) (layer Edge.Cuts) (width 0.15))
 (segment (start 195.045 88.97) (end 195.095 89.02) (width 0.3) (layer B.Cu) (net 4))
 (segment (start 181.35 84.555) (end 181.35 84.35) (width 0.6) (layer B.Cu) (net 8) (status C00000))
 (segment (start 181.35 84.35) (end 181 84) (width 0.6) (layer B.Cu) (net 8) (status 400000))
 (segment (start 181 84) (end 181 74) (width 0.6) (layer B.Cu) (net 8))
 (segment (start 181 74) (end 182.5 72.5) (width 0.6) (layer B.Cu) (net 8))
 (via (at 182.5 72.5) (size 1.4) (drill 0.8) (layers F.Cu B.Cu) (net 8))
 (segment (start 182.5 72.5) (end 184.5 72.5) (width 0.6) (layer F.Cu) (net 8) (status 800000))
 (segment (start 186.75 72.5) (end 188.465 72.5) (width 0.6) (layer F.Cu) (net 8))
 (segment (start 188.465 72.5) (end 190.465 74.5) (width 0.6) (layer F.Cu) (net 8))
 (segment (start 184.5 72.5) (end 186.75 72.5) (width 0.6) (layer F.Cu) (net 8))
 (segment (start 181.35 87.095) (end 182.405 87.095) (width 0.6) (layer B.Cu) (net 9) (status 400000))
 (segment (start 182.5 82.5) (end 184.5 82.5) (width 0.6) (layer F.Cu) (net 9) (status 800000))
 (via (at 182.5 82.5) (size 1.4) (drill 0.8) (layers F.Cu B.Cu) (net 9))
 (segment (start 183 83) (end 182.5 82.5) (width 0.6) (layer B.Cu) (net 9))
 (segment (start 183 86.5) (end 183 83) (width 0.6) (layer B.Cu) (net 9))
 (segment (start 182.405 87.095) (end 183 86.5) (width 0.6) (layer B.Cu) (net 9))
 (segment (start 186.75 82.5) (end 188.465 82.5) (width 0.6) (layer F.Cu) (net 9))
 (segment (start 188.465 82.5) (end 190.465 80.5) (width 0.6) (layer F.Cu) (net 9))
 (segment (start 184.5 82.5) (end 186.75 82.5) (width 0.6) (layer F.Cu) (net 9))
 (segment (start 182.5 75.5) (end 184.5 75.5) (width 0.6) (layer F.Cu) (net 10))
 (segment (start 173.5 76.2) (end 181.8 76.2) (width 1) (layer F.Cu) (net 10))
 (segment (start 192 75.5) (end 198 81.5) (width 1) (layer B.Cu) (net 10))
 (segment (start 182.5 75.5) (end 192 75.5) (width 1) (layer B.Cu) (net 10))
 (via (at 182.5 75.5) (size 1.4) (drill 0.8) (layers F.Cu B.Cu) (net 10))
 (segment (start 181.8 76.2) (end 182.5 75.5) (width 1) (layer F.Cu) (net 10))
 (segment (start 185.5 75.5) (end 185.5 79.5) (width 0.6) (layer F.Cu) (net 10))
 (segment (start 184.5 75.5) (end 185.5 75.5) (width 0.6) (layer F.Cu) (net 10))
 (segment (start 185.5 75.5) (end 186.75 75.5) (width 0.6) (layer F.Cu) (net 10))
 (segment (start 184.5 79.5) (end 185.5 79.5) (width 0.6) (layer F.Cu) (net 10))
 (segment (start 185.5 79.5) (end 186.75 79.5) (width 0.6) (layer F.Cu) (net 10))
 (segment (start 195.045 91.97) (end 195.095 91.92) (width 0.3) (layer B.Cu) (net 12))
 (segment (start 186.75 95.5) (end 188.465 95.5) (width 0.6) (layer F.Cu) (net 13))
 (segment (start 188.465 95.5) (end 190.465 97.5) (width 0.6) (layer F.Cu) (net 13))
 (segment (start 184.5 95.5) (end 186.75 95.5) (width 0.6) (layer F.Cu) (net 13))
 (segment (start 183 105.5) (end 184.5 105.5) (width 0.6) (layer F.Cu) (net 14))
 (segment (start 181.33 103.83) (end 183 105.5) (width 0.6) (layer F.Cu) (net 14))
 (segment (start 186.75 105.5) (end 188.465 105.5) (width 0.6) (layer F.Cu) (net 14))
 (segment (start 188.465 105.5) (end 190.465 103.5) (width 0.6) (layer F.Cu) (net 14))
 (segment (start 184.5 105.5) (end 186.75 105.5) (width 0.6) (layer F.Cu) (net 14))
 (segment (start 185.5 98.5) (end 185.5 102.5) (width 0.6) (layer F.Cu) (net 15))
 (segment (start 184.5 98.5) (end 185.5 98.5) (width 0.6) (layer F.Cu) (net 15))
 (segment (start 185.5 98.5) (end 186.75 98.5) (width 0.6) (layer F.Cu) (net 15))
 (segment (start 184.5 102.5) (end 185.5 102.5) (width 0.6) (layer F.Cu) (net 15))
 (segment (start 185.5 102.5) (end 186.75 102.5) (width 0.6) (layer F.Cu) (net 15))
 (segment (start 194.335 78.59) (end 193.59 78.59) (width 0.3) (layer F.Cu) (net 18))
 (segment (start 193.25 78) (end 192.75 77.5) (width 0.3) (layer F.Cu) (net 18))
 (segment (start 193.25 78.25) (end 193.25 78) (width 0.3) (layer F.Cu) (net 18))
 (segment (start 193.59 78.59) (end 193.25 78.25) (width 0.3) (layer F.Cu) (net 18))
 (segment (start 194.335 72.59) (end 193.41 72.59) (width 0.3) (layer F.Cu) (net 18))
 (segment (start 192.75 77.5) (end 186.95 77.5) (width 0.3) (layer F.Cu) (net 18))
 (segment (start 193.25 77) (end 192.75 77.5) (width 0.3) (layer F.Cu) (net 18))
 (segment (start 193.25 72.75) (end 193.25 77) (width 0.3) (layer F.Cu) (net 18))
 (segment (start 193.41 72.59) (end 193.25 72.75) (width 0.3) (layer F.Cu) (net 18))
 (segment (start 181.35 85.825) (end 179.325 85.825) (width 0.6) (layer B.Cu) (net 20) (status 400000))
 (segment (start 181.75 77.5) (end 184.05 77.5) (width 0.6) (layer F.Cu) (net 20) (status 800000))
 (segment (start 179.25 80) (end 181.75 77.5) (width 0.6) (layer F.Cu) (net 20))
 (segment (start 179.25 85.75) (end 179.25 80) (width 0.6) (layer F.Cu) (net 20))
 (via (at 179.25 85.75) (size 1.4) (drill 0.8) (layers F.Cu B.Cu) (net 20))
 (segment (start 179.325 85.825) (end 179.25 85.75) (width 0.6) (layer B.Cu) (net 20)))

